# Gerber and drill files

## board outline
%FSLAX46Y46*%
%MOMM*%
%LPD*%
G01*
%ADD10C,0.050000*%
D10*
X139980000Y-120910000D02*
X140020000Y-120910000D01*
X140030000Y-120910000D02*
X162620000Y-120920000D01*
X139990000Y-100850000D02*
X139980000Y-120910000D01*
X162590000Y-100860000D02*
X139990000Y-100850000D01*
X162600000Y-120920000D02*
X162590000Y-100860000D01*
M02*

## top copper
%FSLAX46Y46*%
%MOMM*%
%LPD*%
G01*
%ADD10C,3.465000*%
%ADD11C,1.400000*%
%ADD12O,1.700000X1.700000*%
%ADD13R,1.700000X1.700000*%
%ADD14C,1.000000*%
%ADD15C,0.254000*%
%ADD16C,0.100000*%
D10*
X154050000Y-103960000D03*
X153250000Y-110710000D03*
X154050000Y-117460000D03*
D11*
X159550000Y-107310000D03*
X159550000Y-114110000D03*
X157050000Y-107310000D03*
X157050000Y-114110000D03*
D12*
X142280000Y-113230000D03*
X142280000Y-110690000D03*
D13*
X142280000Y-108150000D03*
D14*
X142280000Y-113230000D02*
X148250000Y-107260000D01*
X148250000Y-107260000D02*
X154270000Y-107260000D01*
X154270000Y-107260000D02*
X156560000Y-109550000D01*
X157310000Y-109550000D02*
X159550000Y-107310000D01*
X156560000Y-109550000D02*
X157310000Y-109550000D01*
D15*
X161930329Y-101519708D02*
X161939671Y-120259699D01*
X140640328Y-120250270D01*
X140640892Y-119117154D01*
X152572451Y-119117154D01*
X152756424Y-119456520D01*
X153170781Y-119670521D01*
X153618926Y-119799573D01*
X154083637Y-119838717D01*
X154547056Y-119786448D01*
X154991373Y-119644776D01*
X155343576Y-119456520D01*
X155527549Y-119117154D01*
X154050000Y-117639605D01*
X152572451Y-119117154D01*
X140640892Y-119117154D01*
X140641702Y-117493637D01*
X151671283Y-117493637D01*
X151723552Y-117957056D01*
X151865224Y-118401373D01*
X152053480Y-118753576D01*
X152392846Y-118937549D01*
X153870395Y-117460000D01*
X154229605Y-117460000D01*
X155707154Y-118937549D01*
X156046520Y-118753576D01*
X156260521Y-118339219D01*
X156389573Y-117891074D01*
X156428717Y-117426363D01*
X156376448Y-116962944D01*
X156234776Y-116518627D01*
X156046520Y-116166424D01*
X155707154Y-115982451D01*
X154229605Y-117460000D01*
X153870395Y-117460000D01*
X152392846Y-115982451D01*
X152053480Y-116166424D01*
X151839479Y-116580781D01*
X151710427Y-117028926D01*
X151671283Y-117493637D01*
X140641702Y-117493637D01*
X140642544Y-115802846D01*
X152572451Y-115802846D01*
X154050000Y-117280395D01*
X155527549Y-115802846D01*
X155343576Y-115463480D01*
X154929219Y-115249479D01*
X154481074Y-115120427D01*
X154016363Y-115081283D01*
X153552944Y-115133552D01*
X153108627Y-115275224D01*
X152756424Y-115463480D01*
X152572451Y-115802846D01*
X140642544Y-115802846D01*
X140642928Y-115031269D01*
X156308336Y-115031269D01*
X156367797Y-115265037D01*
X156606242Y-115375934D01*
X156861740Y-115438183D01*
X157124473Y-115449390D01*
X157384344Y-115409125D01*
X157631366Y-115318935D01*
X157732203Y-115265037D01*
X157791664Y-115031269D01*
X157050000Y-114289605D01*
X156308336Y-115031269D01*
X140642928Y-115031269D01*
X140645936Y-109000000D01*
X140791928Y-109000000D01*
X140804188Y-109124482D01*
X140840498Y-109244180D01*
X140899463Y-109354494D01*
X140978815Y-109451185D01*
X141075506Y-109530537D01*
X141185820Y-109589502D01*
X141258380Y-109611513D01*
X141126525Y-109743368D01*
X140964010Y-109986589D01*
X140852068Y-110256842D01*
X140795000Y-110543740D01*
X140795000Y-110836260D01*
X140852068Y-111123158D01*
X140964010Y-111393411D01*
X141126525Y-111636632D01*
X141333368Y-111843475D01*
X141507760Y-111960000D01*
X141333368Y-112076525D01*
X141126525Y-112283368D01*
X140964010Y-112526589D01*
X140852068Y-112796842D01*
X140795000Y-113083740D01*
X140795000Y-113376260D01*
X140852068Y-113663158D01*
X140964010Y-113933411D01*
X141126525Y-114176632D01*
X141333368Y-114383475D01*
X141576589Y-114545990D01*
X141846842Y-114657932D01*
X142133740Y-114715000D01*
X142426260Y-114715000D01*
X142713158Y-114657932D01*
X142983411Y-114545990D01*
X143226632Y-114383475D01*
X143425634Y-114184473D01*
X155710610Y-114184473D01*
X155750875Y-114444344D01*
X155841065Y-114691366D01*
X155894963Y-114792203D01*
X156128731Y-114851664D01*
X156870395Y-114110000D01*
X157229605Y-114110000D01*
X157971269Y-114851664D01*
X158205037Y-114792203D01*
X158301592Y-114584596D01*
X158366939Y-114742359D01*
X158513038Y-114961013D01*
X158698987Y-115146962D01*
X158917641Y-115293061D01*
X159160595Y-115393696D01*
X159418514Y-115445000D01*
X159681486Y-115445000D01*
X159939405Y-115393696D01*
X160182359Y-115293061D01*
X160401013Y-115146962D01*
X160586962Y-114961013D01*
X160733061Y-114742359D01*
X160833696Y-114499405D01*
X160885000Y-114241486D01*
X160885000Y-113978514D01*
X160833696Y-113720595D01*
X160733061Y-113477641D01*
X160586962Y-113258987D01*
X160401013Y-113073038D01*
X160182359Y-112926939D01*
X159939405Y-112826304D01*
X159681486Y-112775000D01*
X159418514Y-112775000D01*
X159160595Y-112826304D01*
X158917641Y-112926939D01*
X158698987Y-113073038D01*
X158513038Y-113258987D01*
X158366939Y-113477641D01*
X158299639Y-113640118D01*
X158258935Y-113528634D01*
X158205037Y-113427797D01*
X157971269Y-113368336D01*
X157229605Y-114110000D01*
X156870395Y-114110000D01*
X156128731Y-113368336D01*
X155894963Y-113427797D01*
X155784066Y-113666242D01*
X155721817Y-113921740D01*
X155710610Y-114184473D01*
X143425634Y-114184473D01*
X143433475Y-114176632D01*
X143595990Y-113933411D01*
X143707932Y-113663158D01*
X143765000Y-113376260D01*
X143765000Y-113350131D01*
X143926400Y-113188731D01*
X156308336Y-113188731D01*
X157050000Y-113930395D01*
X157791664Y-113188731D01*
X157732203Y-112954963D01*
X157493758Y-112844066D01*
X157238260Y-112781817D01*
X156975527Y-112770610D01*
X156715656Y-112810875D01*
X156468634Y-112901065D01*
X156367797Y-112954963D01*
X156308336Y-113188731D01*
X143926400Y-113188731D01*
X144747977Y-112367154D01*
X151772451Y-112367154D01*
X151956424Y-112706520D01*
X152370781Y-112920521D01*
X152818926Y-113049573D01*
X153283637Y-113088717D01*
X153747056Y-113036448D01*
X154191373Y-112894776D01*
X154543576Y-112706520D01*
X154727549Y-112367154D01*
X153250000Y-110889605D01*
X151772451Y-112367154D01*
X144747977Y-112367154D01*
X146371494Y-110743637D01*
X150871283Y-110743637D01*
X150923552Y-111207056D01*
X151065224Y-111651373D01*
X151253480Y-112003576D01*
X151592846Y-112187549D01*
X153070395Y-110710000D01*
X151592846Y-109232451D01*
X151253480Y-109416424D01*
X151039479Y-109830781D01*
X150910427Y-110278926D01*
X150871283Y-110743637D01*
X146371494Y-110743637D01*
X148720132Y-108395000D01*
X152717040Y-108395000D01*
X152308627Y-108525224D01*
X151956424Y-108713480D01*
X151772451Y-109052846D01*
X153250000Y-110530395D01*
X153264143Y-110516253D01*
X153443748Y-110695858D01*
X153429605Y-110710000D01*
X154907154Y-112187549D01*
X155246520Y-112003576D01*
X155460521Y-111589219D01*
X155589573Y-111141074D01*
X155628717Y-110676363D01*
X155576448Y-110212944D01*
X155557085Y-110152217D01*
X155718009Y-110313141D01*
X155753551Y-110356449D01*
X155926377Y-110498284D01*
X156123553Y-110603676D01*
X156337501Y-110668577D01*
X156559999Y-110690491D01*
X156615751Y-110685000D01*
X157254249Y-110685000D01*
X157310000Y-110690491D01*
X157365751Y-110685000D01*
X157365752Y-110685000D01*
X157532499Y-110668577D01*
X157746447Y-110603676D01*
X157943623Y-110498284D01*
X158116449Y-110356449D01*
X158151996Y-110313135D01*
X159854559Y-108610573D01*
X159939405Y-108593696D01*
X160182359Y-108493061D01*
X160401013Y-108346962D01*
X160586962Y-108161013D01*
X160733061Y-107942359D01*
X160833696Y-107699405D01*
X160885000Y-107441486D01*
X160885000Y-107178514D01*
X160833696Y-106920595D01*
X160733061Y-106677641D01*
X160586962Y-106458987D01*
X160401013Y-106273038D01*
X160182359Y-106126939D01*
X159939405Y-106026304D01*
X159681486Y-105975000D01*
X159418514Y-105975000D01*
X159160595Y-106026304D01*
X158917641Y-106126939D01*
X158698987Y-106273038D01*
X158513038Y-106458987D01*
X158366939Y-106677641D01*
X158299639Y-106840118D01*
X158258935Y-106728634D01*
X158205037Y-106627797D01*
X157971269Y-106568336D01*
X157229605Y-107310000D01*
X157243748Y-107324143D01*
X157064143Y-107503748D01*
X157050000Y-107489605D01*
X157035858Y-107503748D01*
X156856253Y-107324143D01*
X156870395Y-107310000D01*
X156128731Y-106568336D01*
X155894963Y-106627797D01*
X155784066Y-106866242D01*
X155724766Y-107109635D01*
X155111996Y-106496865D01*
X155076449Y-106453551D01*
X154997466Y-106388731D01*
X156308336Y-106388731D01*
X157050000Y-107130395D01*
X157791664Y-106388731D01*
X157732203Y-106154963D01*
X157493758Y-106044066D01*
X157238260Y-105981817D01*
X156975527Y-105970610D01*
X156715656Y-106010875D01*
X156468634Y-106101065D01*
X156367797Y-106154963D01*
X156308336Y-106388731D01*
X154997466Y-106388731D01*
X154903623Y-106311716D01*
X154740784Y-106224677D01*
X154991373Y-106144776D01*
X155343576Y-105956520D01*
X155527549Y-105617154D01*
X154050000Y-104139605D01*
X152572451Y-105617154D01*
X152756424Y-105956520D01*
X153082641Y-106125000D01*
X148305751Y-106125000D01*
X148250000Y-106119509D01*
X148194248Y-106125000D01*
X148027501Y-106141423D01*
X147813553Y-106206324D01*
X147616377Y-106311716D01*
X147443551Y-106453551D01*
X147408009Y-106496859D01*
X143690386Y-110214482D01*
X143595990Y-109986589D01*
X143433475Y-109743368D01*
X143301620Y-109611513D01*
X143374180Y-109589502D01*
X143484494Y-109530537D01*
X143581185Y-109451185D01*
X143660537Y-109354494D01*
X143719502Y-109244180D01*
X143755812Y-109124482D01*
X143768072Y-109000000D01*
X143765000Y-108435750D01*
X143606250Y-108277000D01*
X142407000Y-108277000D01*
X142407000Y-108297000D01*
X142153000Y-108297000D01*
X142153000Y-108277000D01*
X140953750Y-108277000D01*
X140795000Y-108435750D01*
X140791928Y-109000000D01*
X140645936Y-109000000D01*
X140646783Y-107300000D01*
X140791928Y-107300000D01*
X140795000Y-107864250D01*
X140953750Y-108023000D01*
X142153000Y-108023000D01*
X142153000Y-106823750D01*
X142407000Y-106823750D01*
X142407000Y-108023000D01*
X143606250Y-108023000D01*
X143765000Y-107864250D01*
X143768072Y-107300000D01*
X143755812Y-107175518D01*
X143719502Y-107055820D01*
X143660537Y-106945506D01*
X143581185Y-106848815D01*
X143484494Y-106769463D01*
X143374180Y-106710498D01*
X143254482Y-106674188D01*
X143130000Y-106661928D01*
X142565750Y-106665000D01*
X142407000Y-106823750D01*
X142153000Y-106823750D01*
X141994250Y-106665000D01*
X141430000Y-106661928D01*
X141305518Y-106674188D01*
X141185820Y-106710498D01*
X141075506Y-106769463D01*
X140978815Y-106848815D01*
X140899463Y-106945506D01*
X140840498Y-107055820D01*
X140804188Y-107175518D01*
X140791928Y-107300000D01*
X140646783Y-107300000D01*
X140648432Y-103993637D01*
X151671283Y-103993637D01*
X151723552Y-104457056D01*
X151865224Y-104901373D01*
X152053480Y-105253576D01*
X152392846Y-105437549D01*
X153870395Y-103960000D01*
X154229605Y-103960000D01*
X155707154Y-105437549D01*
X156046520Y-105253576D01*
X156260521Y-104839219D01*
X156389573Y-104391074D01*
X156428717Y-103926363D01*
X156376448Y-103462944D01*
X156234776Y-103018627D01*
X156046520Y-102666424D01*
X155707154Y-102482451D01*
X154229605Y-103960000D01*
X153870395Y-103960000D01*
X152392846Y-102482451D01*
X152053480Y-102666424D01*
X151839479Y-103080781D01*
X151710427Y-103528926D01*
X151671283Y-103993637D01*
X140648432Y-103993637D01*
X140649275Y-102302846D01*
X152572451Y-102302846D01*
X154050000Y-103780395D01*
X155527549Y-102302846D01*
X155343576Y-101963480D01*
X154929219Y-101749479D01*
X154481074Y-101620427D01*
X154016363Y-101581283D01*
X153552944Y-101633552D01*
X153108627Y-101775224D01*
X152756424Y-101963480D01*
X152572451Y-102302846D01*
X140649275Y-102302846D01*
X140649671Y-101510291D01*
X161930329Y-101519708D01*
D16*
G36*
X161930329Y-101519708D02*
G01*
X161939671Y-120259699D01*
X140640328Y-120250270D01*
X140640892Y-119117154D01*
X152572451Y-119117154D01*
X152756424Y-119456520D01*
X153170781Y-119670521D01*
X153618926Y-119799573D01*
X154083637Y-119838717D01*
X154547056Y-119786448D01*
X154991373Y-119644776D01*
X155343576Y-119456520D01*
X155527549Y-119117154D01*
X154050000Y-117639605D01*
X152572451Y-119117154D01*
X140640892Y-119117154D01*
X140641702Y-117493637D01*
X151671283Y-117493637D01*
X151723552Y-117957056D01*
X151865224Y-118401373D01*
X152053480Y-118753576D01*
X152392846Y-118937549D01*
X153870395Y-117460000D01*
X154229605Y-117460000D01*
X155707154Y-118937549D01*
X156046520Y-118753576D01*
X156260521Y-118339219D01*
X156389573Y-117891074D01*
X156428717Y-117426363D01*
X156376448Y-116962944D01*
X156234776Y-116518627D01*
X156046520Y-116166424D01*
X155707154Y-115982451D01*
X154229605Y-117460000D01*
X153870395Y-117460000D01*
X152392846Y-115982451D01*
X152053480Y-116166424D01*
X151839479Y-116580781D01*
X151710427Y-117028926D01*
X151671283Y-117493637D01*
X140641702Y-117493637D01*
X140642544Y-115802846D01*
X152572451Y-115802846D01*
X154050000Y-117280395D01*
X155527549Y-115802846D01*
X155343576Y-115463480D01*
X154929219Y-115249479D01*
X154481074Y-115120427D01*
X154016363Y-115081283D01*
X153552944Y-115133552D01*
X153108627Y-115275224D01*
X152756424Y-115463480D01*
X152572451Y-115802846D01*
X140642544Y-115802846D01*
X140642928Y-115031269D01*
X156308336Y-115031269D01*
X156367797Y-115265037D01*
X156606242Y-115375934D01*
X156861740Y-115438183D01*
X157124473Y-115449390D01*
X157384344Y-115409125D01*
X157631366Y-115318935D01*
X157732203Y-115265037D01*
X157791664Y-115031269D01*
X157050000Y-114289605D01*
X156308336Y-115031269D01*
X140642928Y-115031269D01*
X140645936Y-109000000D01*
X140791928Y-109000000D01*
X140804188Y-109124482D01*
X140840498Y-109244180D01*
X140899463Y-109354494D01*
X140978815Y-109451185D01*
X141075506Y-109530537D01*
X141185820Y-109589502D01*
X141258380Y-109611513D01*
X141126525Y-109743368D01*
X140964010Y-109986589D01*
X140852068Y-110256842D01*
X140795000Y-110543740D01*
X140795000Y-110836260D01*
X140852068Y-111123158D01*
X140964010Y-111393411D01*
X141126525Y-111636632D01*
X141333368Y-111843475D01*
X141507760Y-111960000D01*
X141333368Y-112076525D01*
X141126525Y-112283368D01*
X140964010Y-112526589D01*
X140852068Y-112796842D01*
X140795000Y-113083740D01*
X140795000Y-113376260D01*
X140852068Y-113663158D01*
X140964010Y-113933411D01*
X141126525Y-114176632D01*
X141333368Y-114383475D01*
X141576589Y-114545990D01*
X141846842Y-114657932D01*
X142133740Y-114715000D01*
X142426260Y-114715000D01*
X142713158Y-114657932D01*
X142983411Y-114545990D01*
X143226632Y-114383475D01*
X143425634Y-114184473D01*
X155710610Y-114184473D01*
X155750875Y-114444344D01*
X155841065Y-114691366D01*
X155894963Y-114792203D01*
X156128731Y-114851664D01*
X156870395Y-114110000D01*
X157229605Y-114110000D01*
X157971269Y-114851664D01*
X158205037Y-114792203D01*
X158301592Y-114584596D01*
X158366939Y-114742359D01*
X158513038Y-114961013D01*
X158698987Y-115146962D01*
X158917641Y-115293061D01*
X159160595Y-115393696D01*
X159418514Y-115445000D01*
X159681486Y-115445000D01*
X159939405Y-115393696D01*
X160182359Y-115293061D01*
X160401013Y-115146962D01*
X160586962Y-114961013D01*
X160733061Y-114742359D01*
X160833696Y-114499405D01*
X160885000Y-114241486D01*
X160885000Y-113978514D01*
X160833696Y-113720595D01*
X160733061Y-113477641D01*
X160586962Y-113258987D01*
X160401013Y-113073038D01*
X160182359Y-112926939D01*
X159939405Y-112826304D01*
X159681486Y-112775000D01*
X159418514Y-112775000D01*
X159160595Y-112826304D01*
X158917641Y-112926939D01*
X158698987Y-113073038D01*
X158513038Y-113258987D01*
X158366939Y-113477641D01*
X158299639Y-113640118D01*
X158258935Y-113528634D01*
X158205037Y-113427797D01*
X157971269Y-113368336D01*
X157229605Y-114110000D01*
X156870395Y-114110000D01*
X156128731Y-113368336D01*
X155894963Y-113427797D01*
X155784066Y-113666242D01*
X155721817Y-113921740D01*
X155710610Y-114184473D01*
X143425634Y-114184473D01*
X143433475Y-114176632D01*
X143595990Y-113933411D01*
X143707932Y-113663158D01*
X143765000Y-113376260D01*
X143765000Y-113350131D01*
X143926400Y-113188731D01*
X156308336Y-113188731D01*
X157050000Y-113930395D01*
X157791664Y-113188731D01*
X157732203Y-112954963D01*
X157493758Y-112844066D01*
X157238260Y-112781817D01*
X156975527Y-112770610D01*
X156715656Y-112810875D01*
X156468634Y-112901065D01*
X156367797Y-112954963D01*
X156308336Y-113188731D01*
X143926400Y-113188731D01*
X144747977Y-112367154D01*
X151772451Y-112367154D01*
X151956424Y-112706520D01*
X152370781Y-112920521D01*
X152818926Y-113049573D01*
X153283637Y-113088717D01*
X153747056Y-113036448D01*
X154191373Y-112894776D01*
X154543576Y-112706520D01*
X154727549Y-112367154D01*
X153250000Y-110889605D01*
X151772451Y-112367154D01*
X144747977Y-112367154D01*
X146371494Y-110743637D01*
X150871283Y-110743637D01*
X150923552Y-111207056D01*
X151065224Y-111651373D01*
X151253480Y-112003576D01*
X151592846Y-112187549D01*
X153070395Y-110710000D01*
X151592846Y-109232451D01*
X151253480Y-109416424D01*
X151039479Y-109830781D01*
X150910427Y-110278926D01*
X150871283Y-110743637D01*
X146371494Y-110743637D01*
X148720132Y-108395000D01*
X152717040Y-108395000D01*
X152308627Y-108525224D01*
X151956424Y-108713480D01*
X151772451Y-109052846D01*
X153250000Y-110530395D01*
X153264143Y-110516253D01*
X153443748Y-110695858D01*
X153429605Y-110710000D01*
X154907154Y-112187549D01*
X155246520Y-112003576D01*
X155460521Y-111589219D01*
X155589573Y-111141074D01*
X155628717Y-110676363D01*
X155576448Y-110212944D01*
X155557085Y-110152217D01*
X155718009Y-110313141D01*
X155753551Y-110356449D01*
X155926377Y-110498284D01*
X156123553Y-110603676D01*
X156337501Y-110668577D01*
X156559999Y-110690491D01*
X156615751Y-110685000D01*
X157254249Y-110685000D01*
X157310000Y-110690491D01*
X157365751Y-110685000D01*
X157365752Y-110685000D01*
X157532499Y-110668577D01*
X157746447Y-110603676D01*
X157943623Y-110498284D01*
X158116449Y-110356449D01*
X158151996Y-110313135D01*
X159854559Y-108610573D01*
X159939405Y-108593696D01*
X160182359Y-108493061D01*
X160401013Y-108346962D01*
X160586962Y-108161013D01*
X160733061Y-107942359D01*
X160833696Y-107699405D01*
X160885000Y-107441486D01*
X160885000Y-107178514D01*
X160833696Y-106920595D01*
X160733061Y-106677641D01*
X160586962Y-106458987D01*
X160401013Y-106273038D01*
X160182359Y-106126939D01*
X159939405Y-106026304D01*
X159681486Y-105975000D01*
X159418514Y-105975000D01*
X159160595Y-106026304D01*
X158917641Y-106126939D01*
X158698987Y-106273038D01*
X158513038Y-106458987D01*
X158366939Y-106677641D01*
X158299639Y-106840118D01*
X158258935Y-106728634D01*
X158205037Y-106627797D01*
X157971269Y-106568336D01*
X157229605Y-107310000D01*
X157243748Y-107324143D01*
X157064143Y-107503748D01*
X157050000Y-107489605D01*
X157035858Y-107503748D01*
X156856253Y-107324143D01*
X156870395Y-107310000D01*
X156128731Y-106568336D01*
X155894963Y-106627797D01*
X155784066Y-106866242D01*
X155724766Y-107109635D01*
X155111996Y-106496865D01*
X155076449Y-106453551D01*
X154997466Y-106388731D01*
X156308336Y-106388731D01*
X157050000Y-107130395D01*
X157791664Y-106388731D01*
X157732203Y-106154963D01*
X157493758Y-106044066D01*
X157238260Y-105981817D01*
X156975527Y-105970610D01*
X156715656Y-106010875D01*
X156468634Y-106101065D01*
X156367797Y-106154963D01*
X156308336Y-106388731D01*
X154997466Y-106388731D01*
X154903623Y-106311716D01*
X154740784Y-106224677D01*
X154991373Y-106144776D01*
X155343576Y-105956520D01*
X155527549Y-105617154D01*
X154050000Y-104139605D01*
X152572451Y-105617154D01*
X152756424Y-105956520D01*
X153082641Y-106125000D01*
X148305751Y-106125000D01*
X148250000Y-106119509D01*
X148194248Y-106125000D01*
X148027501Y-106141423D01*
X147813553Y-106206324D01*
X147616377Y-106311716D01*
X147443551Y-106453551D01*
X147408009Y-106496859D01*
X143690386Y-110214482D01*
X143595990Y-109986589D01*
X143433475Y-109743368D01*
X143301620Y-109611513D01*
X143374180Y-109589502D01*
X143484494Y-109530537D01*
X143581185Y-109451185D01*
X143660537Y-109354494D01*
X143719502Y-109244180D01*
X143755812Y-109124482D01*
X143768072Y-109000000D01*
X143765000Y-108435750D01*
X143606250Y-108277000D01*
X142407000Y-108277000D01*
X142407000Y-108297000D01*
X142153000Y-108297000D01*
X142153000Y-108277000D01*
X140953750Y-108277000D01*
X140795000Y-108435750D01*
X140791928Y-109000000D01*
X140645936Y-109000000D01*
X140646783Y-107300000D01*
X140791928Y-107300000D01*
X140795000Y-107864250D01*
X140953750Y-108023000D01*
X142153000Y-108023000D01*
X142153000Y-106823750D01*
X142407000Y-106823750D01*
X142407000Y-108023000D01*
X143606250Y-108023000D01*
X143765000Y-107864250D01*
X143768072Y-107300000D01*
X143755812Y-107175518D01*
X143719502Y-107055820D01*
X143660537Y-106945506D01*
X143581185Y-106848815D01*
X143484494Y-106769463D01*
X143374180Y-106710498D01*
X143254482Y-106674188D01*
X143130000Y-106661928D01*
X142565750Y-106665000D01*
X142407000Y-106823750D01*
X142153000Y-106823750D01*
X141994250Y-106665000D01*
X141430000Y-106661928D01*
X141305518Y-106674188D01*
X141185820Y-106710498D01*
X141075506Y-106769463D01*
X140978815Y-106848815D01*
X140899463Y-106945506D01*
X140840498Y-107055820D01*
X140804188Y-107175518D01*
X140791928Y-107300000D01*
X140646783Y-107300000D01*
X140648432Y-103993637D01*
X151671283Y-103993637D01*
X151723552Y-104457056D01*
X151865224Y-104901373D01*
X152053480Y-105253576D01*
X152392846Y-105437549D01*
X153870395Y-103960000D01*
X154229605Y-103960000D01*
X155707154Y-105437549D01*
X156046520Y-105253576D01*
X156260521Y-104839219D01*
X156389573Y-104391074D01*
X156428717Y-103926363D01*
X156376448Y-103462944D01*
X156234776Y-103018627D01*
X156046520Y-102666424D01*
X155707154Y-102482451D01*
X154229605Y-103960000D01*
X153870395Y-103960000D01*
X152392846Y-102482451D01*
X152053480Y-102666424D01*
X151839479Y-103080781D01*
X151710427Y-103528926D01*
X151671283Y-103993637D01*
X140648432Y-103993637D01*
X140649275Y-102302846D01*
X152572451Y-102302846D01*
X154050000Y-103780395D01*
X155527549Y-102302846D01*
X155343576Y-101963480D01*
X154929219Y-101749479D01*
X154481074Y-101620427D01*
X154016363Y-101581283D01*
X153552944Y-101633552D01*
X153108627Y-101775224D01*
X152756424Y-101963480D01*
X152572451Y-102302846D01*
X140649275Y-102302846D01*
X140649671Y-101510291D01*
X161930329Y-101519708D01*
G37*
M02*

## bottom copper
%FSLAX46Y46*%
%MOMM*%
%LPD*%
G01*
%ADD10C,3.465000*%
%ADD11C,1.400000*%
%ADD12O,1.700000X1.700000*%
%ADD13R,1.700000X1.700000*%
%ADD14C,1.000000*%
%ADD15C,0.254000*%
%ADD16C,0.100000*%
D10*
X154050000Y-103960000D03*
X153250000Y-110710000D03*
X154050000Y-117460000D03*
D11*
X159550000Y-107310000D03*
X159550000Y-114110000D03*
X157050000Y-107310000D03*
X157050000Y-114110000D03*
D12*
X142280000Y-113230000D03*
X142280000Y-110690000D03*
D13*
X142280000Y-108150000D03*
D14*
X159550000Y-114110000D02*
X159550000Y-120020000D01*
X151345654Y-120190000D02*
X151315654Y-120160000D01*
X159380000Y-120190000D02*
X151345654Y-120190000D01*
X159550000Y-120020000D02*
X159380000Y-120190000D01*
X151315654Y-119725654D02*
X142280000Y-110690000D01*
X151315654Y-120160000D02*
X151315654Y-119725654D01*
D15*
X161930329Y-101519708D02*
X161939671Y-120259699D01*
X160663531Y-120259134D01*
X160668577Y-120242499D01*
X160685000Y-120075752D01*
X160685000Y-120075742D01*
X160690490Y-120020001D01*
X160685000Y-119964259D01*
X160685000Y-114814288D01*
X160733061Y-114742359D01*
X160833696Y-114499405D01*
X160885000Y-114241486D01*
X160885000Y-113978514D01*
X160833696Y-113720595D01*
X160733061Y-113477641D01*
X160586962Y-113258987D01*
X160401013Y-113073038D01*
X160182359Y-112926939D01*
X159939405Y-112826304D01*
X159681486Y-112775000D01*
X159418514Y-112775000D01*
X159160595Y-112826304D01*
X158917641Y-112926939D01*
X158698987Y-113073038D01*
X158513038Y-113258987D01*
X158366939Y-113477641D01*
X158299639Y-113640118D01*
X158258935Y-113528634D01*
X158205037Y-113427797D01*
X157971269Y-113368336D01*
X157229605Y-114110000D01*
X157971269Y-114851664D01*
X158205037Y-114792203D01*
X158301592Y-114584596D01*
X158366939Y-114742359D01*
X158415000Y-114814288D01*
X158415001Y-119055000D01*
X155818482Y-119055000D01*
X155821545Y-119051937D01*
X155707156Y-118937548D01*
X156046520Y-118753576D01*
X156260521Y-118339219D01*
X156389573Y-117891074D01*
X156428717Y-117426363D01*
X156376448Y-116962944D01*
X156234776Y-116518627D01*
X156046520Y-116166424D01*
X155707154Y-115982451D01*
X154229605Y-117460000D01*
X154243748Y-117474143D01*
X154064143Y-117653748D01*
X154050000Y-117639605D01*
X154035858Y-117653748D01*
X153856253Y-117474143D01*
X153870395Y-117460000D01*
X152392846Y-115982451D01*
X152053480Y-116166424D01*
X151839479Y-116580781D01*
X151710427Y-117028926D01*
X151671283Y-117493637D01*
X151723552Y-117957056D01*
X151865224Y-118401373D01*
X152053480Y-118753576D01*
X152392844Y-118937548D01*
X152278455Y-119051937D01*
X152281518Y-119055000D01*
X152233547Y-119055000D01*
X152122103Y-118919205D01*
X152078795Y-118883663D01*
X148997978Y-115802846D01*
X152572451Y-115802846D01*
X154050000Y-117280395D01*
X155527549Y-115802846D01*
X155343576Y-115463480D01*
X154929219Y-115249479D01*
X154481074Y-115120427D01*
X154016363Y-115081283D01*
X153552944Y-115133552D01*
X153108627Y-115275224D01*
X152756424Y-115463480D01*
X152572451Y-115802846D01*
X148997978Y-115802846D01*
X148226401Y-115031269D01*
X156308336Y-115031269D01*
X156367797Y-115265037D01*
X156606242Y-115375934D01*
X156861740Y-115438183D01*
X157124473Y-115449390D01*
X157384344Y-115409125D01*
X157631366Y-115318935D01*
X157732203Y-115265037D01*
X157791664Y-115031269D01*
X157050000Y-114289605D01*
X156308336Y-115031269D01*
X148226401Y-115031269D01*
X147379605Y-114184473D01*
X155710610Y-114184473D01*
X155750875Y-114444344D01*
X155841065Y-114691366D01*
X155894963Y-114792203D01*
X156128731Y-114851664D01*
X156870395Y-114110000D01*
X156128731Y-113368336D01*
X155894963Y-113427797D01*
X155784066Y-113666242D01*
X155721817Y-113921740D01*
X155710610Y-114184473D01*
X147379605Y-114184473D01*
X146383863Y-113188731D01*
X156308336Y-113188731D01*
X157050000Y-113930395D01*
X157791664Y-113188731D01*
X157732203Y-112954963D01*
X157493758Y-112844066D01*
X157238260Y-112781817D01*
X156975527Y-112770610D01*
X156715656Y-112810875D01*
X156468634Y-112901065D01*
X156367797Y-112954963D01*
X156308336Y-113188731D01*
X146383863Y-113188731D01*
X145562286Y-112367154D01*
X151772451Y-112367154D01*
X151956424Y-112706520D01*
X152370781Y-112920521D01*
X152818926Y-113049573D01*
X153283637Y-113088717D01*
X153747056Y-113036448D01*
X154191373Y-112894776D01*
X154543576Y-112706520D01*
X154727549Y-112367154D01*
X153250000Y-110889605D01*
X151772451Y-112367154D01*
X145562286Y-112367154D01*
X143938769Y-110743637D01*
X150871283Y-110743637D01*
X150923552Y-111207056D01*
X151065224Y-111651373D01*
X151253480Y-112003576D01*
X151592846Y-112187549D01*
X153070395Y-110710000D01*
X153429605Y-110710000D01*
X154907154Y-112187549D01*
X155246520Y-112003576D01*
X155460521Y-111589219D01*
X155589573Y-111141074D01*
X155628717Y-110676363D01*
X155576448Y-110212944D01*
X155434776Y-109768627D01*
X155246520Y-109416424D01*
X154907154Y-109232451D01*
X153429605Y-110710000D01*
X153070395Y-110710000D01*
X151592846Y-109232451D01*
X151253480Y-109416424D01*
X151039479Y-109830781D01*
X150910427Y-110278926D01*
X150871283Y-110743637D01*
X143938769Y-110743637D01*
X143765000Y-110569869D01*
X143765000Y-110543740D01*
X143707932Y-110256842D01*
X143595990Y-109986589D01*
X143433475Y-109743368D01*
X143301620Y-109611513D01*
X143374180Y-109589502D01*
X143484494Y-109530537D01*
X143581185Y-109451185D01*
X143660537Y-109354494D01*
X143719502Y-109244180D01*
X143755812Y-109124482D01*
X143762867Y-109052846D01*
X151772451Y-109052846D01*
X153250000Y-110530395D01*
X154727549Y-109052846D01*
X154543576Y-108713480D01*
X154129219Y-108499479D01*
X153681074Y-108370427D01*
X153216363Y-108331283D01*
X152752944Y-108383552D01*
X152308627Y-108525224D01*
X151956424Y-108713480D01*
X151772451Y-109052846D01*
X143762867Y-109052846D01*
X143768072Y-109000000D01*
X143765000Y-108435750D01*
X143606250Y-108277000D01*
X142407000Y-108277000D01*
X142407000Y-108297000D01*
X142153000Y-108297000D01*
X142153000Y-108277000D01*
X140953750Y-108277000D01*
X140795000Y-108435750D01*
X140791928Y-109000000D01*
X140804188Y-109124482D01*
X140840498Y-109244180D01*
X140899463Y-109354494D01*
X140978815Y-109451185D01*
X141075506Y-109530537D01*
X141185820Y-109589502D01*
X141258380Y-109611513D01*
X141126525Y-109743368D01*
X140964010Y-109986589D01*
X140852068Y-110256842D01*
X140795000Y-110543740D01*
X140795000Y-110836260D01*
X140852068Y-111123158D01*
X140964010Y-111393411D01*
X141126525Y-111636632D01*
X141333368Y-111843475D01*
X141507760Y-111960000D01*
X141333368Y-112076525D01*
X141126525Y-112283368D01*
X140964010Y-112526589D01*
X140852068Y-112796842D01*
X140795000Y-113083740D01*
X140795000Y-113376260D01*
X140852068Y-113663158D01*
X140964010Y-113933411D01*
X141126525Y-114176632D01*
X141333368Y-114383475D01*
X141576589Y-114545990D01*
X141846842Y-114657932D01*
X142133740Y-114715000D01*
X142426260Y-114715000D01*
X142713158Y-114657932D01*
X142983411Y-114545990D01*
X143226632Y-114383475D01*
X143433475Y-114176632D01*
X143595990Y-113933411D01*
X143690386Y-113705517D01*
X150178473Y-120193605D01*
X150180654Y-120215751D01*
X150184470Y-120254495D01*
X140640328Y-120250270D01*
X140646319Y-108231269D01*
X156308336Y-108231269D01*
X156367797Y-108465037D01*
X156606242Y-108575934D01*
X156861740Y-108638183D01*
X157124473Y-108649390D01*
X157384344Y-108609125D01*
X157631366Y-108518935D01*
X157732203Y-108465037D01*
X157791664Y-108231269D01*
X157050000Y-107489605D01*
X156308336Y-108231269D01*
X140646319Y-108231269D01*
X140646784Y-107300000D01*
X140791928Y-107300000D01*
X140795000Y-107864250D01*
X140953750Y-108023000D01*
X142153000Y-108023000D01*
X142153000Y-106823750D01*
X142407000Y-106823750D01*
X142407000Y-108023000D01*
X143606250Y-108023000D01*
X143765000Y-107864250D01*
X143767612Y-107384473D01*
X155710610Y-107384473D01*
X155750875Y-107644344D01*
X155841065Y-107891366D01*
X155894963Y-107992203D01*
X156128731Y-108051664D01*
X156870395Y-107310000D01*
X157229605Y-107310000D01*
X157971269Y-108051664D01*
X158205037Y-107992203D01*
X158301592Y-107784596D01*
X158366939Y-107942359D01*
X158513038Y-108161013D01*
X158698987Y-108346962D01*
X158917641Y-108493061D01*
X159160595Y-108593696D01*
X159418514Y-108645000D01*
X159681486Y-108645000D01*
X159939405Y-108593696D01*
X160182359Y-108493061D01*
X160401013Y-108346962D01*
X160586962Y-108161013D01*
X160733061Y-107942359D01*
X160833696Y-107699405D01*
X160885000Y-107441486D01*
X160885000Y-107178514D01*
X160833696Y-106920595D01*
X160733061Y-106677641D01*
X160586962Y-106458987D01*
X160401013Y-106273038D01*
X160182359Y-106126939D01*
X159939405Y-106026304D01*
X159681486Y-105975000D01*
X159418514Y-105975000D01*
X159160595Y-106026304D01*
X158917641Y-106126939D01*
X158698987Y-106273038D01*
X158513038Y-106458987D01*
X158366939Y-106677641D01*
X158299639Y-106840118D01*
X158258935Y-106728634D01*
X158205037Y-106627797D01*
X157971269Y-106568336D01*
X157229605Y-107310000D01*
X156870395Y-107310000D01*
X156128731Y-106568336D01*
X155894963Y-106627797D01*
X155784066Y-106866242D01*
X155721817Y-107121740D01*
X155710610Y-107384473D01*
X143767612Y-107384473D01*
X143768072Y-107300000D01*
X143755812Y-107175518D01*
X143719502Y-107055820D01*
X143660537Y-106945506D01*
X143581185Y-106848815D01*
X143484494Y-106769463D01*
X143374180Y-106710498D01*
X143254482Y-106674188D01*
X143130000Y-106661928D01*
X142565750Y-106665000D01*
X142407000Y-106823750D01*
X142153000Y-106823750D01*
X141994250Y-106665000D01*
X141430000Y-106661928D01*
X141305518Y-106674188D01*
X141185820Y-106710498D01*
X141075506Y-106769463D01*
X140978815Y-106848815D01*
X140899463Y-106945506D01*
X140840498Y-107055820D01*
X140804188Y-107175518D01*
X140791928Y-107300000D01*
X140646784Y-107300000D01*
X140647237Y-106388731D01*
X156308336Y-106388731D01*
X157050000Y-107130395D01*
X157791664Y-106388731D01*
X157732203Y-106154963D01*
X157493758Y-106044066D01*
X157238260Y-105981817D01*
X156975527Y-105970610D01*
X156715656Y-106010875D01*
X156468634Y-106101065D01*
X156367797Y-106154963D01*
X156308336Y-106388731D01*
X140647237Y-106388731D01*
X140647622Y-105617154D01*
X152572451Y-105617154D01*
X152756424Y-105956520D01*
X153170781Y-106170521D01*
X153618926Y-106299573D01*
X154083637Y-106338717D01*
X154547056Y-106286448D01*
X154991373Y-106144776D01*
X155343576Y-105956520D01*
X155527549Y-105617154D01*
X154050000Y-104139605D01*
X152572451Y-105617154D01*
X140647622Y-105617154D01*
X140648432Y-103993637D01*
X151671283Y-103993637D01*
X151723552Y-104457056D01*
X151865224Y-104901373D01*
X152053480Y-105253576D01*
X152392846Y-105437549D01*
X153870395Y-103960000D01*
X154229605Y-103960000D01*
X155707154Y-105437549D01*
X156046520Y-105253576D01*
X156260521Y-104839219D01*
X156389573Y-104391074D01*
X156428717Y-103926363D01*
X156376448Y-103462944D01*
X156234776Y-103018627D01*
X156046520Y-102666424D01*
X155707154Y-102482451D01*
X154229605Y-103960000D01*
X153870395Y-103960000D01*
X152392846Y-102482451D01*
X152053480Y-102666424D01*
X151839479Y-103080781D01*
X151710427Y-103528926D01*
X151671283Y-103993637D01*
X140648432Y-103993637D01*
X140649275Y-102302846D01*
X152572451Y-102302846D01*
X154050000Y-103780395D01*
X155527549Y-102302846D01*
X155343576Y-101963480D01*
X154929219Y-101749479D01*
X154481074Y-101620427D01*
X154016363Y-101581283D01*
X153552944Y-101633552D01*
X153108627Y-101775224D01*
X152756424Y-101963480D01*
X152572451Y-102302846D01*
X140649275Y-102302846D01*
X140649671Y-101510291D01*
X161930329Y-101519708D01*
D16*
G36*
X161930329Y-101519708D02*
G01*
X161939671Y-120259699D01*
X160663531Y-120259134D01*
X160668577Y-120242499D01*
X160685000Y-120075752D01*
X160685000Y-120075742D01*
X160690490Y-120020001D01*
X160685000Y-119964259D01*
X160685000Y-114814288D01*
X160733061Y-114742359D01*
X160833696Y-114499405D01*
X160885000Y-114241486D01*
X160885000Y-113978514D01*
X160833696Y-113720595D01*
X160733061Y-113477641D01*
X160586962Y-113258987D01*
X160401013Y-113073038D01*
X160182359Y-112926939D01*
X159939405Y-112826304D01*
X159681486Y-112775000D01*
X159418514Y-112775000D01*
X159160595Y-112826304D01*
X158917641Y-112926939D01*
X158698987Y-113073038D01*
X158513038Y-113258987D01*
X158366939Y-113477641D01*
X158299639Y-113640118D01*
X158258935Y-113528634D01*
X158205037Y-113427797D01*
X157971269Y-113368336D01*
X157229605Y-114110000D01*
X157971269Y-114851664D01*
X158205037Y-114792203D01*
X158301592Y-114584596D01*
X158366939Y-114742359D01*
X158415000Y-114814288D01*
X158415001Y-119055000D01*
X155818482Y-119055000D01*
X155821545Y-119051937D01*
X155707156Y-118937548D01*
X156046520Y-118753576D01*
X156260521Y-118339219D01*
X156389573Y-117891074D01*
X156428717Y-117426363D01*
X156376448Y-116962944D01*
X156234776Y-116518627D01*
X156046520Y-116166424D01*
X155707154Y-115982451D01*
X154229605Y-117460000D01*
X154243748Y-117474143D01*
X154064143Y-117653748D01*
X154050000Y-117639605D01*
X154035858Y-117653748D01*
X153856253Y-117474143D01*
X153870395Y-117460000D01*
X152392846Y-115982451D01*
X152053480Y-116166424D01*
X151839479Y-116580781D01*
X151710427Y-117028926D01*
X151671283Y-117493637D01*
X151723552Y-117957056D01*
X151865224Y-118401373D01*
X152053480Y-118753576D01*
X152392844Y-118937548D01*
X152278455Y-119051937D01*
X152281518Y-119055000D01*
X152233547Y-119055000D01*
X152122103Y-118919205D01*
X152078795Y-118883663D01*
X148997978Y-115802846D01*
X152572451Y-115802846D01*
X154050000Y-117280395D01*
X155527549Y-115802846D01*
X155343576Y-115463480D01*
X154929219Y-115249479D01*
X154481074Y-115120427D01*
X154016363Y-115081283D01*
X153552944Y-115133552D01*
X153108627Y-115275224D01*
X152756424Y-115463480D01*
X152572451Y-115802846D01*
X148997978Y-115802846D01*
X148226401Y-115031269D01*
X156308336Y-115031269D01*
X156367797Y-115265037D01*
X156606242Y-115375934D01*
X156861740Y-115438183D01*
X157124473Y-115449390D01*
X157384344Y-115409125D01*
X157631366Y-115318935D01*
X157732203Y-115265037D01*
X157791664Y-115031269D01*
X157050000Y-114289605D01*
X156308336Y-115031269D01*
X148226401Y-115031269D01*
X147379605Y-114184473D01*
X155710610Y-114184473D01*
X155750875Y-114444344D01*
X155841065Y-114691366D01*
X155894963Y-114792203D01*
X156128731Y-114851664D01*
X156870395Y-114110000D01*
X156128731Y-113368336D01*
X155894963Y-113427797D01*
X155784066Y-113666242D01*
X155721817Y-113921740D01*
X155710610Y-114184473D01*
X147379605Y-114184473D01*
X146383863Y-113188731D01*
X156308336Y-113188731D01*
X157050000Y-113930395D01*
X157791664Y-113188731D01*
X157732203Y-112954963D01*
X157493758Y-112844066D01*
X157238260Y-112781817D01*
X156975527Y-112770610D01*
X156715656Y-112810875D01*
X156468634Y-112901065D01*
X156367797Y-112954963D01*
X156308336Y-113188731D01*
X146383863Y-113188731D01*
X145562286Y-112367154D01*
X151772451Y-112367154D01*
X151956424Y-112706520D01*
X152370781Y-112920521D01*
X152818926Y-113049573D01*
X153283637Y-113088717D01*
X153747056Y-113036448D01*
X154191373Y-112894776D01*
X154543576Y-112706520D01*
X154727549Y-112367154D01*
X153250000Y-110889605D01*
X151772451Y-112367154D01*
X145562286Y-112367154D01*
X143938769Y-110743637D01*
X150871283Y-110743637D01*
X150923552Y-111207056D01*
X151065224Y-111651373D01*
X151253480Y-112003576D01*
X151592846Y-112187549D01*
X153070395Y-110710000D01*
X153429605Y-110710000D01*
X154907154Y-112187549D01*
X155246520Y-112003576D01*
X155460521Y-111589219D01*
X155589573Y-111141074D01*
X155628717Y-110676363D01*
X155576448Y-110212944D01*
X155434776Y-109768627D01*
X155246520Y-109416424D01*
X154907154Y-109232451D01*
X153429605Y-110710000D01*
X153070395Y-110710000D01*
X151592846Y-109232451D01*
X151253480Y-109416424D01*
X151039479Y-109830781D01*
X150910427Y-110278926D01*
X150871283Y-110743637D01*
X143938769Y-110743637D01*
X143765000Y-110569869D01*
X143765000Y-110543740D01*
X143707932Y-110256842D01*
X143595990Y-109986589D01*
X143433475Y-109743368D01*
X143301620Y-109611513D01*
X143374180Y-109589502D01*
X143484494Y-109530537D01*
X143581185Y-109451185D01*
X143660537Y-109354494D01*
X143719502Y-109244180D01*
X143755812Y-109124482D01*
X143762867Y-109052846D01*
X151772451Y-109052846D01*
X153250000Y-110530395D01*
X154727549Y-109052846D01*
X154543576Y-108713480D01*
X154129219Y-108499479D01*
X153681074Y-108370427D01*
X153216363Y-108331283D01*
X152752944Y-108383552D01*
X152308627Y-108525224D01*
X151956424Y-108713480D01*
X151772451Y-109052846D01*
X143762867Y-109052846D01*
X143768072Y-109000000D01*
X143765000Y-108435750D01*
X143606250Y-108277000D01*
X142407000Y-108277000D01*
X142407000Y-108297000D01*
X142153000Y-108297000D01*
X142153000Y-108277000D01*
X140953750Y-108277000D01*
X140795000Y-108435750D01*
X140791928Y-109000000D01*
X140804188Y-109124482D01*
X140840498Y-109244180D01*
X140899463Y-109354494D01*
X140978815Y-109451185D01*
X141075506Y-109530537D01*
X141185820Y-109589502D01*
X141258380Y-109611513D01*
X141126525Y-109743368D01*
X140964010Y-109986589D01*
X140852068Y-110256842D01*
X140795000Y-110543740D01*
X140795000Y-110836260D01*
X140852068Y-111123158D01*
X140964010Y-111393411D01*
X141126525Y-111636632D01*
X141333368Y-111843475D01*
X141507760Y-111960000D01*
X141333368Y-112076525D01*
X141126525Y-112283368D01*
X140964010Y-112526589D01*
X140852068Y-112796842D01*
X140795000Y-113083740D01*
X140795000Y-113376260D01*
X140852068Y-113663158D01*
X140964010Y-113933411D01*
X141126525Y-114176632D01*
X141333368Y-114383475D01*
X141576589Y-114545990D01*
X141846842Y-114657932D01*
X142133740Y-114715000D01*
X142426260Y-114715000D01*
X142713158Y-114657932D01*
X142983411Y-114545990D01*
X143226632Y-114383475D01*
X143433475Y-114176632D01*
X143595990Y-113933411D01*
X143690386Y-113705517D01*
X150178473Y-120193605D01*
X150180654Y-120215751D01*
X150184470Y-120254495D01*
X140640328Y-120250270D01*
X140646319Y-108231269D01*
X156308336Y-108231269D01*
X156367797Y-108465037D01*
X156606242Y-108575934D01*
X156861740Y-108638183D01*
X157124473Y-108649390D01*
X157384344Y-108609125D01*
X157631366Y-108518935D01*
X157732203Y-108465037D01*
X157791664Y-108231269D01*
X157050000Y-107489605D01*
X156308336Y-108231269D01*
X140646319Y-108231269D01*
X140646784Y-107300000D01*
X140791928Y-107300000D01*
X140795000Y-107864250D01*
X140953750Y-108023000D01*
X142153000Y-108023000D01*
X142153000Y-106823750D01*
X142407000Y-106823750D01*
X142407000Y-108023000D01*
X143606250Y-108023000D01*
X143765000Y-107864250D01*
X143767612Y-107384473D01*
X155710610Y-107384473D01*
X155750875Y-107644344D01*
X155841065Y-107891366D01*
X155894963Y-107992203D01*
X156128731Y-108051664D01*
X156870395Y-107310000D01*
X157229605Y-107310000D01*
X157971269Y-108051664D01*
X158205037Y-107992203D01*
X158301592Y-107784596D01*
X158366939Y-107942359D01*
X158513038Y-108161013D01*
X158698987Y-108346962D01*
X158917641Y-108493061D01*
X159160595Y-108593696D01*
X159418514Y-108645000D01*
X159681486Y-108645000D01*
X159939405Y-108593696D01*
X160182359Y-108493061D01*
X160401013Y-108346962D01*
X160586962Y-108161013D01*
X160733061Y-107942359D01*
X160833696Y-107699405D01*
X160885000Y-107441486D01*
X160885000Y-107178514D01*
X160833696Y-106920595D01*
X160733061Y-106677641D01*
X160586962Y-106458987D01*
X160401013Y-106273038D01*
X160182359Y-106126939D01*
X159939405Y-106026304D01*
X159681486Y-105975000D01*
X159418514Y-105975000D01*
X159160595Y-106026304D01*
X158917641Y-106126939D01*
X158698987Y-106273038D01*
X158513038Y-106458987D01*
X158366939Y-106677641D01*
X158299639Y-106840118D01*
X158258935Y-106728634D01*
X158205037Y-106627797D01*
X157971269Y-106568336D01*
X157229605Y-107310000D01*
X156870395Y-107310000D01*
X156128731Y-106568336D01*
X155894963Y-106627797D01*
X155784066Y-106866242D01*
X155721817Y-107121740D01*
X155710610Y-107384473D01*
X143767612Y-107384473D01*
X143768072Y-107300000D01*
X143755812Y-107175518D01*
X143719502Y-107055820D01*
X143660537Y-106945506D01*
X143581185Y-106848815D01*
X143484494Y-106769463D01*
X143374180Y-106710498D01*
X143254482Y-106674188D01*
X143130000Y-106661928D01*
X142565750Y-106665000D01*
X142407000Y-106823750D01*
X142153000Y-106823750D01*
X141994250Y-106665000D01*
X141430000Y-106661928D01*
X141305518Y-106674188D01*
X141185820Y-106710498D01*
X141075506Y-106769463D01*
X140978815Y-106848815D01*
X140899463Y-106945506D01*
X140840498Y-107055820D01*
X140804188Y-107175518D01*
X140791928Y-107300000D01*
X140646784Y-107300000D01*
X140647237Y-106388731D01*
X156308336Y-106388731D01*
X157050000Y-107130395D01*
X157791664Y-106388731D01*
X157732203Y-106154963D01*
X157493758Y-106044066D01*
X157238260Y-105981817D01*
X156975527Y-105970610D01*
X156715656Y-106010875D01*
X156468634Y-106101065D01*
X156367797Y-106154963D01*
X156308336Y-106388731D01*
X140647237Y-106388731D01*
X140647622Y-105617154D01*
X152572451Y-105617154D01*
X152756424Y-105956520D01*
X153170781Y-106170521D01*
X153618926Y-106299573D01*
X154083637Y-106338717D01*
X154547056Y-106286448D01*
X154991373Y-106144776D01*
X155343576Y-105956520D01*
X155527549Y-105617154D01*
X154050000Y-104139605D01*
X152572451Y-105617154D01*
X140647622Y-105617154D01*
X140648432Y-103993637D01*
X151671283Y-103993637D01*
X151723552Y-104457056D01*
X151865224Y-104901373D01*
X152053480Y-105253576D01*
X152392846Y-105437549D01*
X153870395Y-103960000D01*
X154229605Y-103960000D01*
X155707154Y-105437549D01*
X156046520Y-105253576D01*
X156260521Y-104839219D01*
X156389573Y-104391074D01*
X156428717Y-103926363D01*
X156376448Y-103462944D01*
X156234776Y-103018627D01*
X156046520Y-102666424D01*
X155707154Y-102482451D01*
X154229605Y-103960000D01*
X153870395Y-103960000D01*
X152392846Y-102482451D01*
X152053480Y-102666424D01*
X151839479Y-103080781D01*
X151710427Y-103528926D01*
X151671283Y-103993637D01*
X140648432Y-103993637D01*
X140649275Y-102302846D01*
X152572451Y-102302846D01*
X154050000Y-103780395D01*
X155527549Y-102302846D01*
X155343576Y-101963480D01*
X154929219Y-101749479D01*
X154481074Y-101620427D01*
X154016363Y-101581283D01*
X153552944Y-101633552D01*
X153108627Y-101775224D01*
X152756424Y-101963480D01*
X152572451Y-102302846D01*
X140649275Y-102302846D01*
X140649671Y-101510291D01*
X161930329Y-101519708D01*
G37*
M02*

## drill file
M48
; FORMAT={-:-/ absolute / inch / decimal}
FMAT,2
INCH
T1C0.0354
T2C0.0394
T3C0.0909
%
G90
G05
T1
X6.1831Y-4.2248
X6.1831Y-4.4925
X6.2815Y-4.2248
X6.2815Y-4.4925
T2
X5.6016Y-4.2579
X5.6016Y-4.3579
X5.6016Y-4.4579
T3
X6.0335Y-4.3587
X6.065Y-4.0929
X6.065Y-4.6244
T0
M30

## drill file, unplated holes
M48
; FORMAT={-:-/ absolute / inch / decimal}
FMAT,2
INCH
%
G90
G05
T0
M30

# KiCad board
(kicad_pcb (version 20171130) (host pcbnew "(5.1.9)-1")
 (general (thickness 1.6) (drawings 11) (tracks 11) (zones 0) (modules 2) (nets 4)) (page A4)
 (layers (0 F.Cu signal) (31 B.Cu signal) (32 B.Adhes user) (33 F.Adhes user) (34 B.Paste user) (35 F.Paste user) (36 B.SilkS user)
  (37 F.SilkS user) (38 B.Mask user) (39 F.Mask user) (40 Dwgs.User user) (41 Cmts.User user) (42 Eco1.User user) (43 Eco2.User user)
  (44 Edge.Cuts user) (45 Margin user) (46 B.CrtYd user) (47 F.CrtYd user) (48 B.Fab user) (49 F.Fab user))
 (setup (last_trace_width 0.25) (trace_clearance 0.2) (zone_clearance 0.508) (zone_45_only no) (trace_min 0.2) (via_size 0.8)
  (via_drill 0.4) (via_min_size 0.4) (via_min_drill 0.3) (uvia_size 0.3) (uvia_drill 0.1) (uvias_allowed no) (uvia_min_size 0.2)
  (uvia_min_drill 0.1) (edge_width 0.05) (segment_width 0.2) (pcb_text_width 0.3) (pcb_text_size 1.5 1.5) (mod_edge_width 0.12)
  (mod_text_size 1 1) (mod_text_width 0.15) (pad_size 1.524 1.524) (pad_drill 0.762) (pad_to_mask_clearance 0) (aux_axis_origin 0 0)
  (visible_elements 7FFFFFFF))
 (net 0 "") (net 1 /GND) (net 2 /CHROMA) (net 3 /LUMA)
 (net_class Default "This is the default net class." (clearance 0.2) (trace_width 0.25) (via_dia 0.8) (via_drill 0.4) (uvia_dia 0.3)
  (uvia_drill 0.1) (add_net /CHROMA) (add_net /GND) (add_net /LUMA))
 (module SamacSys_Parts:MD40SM (layer F.Cu) (at 157.05 114.11 90)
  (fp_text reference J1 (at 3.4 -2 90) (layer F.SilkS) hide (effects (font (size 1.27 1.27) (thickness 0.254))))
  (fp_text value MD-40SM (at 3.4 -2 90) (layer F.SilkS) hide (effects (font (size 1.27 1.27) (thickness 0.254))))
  (pad MH3 thru_hole circle (at 10.15 -3 180) (size 3.465 3.465) (drill 2.31) (layers *.Cu *.Mask F.SilkS) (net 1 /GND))
  (pad MH2 thru_hole circle (at 3.4 -3.8 180) (size 3.465 3.465) (drill 2.31) (layers *.Cu *.Mask F.SilkS) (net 1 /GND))
  (pad MH1 thru_hole circle (at -3.35 -3 180) (size 3.465 3.465) (drill 2.31) (layers *.Cu *.Mask F.SilkS) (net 1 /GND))
  (pad 4 thru_hole circle (at 6.8 2.5 180) (size 1.4 1.4) (drill 0.9) (layers *.Cu *.Mask F.SilkS) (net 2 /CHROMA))
  (pad 3 thru_hole circle (at 0 2.5 180) (size 1.4 1.4) (drill 0.9) (layers *.Cu *.Mask F.SilkS) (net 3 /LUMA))
  (pad 2 thru_hole circle (at 6.8 0 180) (size 1.4 1.4) (drill 0.9) (layers *.Cu *.Mask F.SilkS) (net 1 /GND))
  (pad 1 thru_hole circle (at 0 0 180) (size 1.4 1.4) (drill 0.9) (layers *.Cu *.Mask F.SilkS) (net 1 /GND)))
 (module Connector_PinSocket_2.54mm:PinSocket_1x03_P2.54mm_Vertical (layer F.Cu) (at 142.28 108.15)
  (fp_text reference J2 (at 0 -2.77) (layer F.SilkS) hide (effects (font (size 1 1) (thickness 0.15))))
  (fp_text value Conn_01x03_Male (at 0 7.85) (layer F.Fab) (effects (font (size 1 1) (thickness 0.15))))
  (pad 3 thru_hole oval (at 0 5.08) (size 1.7 1.7) (drill 1) (layers *.Cu *.Mask) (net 2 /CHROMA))
  (pad 2 thru_hole oval (at 0 2.54) (size 1.7 1.7) (drill 1) (layers *.Cu *.Mask) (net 3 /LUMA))
  (pad 1 thru_hole rect (at 0 0) (size 1.7 1.7) (drill 1) (layers *.Cu *.Mask) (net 1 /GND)))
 (gr_line (start 139.98 120.91) (end 140.02 120.91) (layer Edge.Cuts) (width 0.05))
 (gr_line (start 140.03 120.91) (end 162.62 120.92) (layer Edge.Cuts) (width 0.05))
 (gr_line (start 139.99 100.85) (end 139.98 120.91) (layer Edge.Cuts) (width 0.05))
 (gr_line (start 162.59 100.86) (end 139.99 100.85) (layer Edge.Cuts) (width 0.05))
 (gr_line (start 162.6 120.92) (end 162.59 100.86) (layer Edge.Cuts) (width 0.05))
 (segment (start 142.28 113.23) (end 148.25 107.26) (width 1) (layer F.Cu) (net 2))
 (segment (start 148.25 107.26) (end 154.27 107.26) (width 1) (layer F.Cu) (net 2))
 (segment (start 154.27 107.26) (end 156.56 109.55) (width 1) (layer F.Cu) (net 2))
 (segment (start 157.31 109.55) (end 159.55 107.31) (width 1) (layer F.Cu) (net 2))
 (segment (start 156.56 109.55) (end 157.31 109.55) (width 1) (layer F.Cu) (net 2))
 (segment (start 159.55 114.11) (end 159.55 120.02) (width 1) (layer B.Cu) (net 3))
 (segment (start 151.345654 120.19) (end 151.315654 120.16) (width 1) (layer B.Cu) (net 3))
 (segment (start 159.38 120.19) (end 151.345654 120.19) (width 1) (layer B.Cu) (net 3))
 (segment (start 159.55 120.02) (end 159.38 120.19) (width 1) (layer B.Cu) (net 3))
 (segment (start 151.315654 119.725654) (end 142.28 110.69) (width 1) (layer B.Cu) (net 3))
 (segment (start 151.315654 120.16) (end 151.315654 119.725654) (width 1) (layer B.Cu) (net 3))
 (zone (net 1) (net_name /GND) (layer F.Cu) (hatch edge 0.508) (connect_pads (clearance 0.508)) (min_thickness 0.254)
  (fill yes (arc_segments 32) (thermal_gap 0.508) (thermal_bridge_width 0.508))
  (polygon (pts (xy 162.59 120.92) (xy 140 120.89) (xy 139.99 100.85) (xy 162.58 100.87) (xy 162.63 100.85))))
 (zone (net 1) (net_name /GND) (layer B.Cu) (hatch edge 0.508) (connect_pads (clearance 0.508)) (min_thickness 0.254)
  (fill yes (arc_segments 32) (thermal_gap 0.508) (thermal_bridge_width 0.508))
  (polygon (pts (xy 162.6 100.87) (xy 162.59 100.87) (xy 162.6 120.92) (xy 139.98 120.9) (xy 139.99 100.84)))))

